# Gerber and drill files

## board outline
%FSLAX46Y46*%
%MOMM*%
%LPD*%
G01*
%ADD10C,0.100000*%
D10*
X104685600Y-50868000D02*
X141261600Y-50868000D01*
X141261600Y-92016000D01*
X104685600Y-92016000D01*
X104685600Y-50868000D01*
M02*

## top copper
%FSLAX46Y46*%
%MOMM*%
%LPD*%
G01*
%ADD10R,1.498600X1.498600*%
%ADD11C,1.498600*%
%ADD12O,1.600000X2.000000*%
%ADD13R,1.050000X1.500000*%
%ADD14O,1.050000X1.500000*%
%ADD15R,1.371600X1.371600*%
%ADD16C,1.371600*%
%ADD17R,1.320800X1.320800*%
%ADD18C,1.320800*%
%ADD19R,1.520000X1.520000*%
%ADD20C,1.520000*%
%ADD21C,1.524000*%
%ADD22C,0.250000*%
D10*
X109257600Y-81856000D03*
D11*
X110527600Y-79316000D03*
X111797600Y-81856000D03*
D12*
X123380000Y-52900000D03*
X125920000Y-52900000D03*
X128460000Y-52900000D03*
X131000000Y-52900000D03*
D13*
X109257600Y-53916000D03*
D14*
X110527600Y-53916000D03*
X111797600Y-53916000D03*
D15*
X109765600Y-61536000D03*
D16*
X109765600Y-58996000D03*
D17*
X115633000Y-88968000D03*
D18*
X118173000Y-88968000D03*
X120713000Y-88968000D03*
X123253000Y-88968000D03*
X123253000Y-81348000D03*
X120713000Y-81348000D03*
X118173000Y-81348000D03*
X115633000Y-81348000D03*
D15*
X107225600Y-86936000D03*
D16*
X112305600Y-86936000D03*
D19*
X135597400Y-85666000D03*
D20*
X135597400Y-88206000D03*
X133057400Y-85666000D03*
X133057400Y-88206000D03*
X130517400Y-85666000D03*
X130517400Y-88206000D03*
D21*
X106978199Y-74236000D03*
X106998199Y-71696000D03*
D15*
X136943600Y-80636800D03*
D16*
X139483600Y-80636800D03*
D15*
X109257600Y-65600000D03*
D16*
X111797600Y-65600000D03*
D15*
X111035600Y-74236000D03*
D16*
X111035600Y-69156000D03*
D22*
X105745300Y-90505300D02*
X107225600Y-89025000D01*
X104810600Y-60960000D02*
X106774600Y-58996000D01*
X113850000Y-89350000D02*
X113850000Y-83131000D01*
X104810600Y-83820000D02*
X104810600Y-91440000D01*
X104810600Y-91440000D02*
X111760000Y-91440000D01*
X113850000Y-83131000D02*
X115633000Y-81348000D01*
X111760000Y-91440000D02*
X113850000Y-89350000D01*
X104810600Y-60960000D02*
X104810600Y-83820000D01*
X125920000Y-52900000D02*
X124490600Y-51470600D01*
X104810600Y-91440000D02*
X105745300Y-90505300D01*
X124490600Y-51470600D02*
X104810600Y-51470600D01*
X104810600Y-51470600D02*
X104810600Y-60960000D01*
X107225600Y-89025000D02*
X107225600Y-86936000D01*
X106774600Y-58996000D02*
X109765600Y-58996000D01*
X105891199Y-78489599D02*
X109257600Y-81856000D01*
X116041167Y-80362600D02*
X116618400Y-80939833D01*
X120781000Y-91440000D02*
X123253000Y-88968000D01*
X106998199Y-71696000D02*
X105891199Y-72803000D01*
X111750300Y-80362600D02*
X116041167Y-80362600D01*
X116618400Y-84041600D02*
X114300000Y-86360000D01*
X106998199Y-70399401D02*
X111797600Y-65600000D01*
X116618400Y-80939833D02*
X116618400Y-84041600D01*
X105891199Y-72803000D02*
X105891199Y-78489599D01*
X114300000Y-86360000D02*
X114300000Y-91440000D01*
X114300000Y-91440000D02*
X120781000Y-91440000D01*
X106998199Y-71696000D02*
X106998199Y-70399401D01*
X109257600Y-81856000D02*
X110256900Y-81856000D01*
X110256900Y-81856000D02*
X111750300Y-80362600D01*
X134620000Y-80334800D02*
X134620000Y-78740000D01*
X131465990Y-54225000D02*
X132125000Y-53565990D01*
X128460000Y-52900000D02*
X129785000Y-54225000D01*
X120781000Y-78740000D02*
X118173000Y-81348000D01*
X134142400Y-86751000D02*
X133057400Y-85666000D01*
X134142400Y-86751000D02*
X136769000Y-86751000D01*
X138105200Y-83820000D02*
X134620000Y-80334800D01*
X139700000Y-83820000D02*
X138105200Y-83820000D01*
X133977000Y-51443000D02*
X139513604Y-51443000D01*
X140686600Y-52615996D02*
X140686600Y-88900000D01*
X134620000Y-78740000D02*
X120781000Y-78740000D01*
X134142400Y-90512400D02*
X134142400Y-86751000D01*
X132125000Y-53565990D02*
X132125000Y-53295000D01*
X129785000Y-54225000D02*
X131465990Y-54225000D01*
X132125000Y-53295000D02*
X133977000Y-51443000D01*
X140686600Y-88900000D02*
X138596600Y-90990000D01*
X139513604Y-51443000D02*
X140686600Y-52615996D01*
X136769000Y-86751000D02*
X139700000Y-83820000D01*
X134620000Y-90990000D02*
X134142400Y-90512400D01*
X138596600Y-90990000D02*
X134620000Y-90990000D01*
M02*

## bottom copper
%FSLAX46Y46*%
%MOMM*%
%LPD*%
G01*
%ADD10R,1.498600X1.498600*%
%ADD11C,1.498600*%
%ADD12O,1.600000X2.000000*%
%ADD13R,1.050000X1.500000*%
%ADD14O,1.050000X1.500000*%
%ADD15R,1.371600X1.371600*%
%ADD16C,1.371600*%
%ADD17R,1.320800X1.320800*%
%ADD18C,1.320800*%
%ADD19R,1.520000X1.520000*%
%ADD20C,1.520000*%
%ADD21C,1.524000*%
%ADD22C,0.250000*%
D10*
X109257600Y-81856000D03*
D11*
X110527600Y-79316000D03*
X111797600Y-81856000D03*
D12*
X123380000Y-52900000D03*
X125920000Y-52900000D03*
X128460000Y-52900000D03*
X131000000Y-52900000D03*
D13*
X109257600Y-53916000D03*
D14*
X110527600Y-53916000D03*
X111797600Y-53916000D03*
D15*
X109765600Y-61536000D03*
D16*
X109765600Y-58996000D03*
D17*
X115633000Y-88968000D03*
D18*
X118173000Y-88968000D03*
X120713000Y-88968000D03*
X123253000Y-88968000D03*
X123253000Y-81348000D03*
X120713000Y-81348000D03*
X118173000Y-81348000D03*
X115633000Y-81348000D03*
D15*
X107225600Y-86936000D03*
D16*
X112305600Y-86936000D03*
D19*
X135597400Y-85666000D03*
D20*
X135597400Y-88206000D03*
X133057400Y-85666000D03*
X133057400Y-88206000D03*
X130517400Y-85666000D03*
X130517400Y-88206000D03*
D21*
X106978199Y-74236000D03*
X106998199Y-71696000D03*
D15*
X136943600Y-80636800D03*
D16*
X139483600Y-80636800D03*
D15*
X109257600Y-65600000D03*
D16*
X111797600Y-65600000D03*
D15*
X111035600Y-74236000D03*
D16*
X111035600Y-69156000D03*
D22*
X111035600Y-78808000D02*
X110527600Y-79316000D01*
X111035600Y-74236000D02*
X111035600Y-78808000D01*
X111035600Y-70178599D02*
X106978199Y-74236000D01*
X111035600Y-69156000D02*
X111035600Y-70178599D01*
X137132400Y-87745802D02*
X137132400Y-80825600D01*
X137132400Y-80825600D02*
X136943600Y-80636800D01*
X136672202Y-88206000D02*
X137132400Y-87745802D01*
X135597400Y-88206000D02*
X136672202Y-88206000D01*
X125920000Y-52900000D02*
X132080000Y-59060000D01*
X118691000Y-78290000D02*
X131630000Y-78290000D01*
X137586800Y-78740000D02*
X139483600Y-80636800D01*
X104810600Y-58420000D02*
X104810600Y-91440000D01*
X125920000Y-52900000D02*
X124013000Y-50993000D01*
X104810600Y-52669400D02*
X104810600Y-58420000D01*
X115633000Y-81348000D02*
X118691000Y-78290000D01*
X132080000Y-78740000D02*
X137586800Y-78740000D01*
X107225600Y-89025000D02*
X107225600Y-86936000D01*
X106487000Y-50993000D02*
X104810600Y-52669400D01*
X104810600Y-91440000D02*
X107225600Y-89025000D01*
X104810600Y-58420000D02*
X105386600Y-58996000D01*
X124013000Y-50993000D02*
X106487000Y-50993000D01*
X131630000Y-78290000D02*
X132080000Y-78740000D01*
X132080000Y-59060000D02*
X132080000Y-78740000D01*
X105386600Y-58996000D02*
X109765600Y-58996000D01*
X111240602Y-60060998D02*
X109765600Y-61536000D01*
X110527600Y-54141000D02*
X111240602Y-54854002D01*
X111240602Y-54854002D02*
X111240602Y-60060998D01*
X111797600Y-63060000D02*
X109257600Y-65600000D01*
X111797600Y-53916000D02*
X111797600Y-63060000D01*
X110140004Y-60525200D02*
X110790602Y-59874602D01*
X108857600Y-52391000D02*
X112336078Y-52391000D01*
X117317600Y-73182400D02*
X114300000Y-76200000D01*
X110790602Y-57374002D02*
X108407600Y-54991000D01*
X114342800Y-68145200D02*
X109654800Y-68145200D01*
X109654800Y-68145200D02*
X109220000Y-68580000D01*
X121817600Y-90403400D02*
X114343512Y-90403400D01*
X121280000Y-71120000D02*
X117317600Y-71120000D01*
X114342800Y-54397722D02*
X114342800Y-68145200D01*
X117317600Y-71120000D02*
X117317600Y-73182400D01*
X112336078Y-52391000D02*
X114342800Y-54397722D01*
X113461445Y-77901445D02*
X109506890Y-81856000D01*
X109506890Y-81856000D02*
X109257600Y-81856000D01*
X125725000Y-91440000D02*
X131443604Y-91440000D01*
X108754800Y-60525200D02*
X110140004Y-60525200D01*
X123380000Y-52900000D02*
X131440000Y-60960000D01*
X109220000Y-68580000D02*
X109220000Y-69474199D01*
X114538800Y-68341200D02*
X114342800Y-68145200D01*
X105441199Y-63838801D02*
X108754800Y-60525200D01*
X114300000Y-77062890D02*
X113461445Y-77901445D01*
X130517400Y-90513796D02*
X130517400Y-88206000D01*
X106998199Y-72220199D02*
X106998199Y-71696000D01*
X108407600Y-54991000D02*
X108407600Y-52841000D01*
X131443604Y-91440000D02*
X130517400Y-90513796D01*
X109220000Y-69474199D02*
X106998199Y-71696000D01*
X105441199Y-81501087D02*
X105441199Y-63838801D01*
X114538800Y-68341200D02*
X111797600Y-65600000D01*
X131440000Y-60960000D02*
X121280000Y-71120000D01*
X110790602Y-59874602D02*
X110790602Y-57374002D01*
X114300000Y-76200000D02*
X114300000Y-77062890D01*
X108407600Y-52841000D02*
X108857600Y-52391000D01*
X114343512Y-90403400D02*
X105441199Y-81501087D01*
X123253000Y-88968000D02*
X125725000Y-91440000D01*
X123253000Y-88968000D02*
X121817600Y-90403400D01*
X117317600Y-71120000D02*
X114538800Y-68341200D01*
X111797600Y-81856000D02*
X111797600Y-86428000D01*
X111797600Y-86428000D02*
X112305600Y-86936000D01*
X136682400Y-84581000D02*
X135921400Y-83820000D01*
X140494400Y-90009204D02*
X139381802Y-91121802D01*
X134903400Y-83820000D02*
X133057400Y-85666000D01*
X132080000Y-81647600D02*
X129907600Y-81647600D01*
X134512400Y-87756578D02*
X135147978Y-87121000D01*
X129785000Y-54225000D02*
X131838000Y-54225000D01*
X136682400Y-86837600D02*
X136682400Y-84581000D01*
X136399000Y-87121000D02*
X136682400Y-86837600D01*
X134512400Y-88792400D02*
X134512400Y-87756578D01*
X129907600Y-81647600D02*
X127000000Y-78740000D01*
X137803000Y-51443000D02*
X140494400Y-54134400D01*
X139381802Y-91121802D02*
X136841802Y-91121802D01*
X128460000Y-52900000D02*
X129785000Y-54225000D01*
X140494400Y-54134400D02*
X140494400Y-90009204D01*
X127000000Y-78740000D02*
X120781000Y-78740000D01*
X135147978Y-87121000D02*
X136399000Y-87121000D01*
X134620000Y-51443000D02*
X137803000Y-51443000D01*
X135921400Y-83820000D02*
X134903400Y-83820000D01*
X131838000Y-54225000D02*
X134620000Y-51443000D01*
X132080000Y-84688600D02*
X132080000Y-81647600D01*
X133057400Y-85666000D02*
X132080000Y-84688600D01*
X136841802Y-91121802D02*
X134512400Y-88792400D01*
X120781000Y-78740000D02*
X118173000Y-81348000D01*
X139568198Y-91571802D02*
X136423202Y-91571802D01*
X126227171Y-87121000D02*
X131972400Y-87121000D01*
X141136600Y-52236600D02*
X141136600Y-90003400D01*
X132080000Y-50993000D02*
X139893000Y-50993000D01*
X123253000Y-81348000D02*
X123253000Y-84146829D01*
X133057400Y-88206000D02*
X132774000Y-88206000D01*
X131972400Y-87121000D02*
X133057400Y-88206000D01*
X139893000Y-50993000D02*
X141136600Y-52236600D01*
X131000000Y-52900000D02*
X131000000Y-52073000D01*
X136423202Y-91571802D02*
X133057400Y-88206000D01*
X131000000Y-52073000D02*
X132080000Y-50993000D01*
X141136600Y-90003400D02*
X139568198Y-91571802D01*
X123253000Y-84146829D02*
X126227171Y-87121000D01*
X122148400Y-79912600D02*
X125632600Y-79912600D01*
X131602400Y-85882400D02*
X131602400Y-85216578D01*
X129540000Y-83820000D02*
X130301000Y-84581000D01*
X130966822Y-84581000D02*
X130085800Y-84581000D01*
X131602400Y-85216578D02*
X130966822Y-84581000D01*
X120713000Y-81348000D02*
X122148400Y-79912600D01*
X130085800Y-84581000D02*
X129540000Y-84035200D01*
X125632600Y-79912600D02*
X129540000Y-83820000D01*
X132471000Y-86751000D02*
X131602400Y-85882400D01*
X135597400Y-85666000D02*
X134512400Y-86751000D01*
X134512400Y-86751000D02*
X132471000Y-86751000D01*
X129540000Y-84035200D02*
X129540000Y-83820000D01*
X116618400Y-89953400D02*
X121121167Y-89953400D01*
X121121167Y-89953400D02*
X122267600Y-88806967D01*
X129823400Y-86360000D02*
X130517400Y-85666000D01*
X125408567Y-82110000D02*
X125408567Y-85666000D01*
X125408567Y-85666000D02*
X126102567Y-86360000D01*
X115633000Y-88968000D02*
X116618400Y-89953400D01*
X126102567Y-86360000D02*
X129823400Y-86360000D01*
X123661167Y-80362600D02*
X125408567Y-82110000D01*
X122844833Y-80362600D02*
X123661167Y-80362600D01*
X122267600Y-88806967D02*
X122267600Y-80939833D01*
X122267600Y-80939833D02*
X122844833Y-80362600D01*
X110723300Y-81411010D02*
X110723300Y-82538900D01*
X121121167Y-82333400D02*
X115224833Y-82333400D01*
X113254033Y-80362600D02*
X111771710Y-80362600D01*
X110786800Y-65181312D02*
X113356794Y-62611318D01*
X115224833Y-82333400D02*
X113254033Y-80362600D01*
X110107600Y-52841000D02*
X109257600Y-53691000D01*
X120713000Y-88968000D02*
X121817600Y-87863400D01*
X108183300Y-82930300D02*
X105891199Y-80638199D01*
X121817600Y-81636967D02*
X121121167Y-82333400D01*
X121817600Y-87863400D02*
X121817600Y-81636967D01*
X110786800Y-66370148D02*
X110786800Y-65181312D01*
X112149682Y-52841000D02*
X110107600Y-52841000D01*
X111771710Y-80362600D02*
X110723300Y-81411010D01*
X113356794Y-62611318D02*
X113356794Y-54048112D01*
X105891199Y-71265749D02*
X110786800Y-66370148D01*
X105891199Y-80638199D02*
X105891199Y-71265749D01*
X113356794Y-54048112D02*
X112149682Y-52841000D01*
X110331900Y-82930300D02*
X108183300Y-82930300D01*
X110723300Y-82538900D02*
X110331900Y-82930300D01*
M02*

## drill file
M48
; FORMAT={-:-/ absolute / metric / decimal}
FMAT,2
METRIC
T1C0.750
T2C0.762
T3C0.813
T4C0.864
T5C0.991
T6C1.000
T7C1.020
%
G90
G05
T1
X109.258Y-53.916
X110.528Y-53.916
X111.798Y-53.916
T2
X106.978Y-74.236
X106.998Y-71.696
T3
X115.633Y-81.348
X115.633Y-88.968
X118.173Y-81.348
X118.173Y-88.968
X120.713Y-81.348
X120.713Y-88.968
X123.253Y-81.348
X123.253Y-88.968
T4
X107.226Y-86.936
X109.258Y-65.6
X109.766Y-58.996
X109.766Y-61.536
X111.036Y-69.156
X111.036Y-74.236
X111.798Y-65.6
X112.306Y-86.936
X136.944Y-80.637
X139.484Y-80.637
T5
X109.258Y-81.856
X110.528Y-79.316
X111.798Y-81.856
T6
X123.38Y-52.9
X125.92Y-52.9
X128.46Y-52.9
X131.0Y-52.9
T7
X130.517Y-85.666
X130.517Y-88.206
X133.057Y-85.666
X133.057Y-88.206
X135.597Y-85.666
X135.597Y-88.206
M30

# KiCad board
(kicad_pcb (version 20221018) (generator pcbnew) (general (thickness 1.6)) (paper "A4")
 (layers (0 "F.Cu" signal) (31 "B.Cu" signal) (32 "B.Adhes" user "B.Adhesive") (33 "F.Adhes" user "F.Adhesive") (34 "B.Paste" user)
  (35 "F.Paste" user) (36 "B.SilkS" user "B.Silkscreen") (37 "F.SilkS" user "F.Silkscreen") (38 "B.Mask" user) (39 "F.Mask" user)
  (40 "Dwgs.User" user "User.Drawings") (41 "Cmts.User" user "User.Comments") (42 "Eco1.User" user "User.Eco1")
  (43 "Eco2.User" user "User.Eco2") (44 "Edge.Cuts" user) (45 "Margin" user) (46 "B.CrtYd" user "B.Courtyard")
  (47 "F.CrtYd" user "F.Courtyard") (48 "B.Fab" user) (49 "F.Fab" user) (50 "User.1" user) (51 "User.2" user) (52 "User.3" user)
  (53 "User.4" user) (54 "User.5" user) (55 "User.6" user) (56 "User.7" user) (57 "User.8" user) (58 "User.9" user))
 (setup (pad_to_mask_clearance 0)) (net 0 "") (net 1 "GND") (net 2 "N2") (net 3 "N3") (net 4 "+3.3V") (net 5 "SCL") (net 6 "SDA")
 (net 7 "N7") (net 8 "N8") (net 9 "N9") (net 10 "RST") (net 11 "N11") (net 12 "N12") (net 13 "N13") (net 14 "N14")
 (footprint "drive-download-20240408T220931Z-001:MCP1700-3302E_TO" (layer "F.Cu") (at 111.7976 79.316)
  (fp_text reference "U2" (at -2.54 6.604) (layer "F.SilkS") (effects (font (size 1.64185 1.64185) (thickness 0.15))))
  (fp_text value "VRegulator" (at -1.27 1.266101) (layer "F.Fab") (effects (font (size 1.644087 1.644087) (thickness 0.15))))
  (pad "1" thru_hole rect (at -2.54 2.54) (size 1.4986 1.4986) (drill 0.9906) (layers "*.Cu" "*.Mask") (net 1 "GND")
   (solder_mask_margin 0.102))
  (pad "2" thru_hole circle (at -1.27 0) (size 1.4986 1.4986) (drill 0.9906) (layers "*.Cu" "*.Mask") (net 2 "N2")
   (solder_mask_margin 0.102))
  (pad "3" thru_hole circle (at 0 2.54) (size 1.4986 1.4986) (drill 0.9906) (layers "*.Cu" "*.Mask") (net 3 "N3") (solder_mask_margin 0.102)))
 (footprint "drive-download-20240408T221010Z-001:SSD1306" (layer "F.Cu") (at 127 63.5)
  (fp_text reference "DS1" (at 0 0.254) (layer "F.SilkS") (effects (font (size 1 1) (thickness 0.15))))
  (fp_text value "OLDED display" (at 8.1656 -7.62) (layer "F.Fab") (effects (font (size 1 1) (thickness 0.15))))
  (pad "1" thru_hole oval (at -3.62 -10.6 90) (size 2 1.6) (drill 1) (layers "*.Cu" "*.Mask") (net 1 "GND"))
  (pad "2" thru_hole oval (at -1.08 -10.6 90) (size 2 1.6) (drill 1) (layers "*.Cu" "*.Mask") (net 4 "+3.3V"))
  (pad "3" thru_hole oval (at 1.46 -10.6 90) (size 2 1.6) (drill 1) (layers "*.Cu" "*.Mask") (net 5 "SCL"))
  (pad "4" thru_hole oval (at 4 -10.6 90) (size 2 1.6) (drill 1) (layers "*.Cu" "*.Mask") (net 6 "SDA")))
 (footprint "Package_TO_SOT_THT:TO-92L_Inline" (layer "F.Cu") (at 109.2576 53.916)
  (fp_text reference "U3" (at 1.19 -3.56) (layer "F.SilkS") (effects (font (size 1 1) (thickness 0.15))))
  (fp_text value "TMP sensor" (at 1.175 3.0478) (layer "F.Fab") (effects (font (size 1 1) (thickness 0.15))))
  (pad "1" thru_hole rect (at 0 0) (size 1.05 1.5) (drill 0.75) (layers "*.Cu" "*.Mask") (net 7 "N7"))
  (pad "2" thru_hole oval (at 1.27 0) (size 1.05 1.5) (drill 0.75) (layers "*.Cu" "*.Mask") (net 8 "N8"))
  (pad "3" thru_hole oval (at 2.54 0) (size 1.05 1.5) (drill 0.75) (layers "*.Cu" "*.Mask") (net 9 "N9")))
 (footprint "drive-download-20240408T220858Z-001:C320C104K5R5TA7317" (layer "F.Cu") (at 109.7656 61.536 90)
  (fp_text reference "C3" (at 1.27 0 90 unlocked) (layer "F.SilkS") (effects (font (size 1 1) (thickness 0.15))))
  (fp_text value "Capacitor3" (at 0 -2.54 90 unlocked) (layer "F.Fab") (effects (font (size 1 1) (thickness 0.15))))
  (pad "1" thru_hole rect (at 0 0 90) (size 1.3716 1.3716) (drill 0.8636) (layers "*.Cu" "*.Mask") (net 8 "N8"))
  (pad "2" thru_hole circle (at 2.54 0 90) (size 1.3716 1.3716) (drill 0.8636) (layers "*.Cu" "*.Mask") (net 4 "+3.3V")))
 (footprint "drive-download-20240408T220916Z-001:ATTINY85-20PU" (layer "F.Cu") (at 119.443 85.158 90)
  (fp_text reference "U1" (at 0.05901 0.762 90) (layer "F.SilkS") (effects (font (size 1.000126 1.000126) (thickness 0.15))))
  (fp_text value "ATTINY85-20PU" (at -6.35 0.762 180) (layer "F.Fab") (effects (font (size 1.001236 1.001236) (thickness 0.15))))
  (pad "1" thru_hole rect (at -3.81 -3.81 90) (size 1.3208 1.3208) (drill 0.8128) (layers "*.Cu" "*.Mask") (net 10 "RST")
   (solder_mask_margin 0.102))
  (pad "2" thru_hole circle (at -3.81 -1.27 90) (size 1.3208 1.3208) (drill 0.8128) (layers "*.Cu" "*.Mask") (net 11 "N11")
   (solder_mask_margin 0.102))
  (pad "3" thru_hole circle (at -3.81 1.27 90) (size 1.3208 1.3208) (drill 0.8128) (layers "*.Cu" "*.Mask") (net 7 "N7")
   (solder_mask_margin 0.102))
  (pad "4" thru_hole circle (at -3.81 3.81 90) (size 1.3208 1.3208) (drill 0.8128) (layers "*.Cu" "*.Mask") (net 1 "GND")
   (solder_mask_margin 0.102))
  (pad "5" thru_hole circle (at 3.81 3.81 90) (size 1.3208 1.3208) (drill 0.8128) (layers "*.Cu" "*.Mask") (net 6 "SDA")
   (solder_mask_margin 0.102))
  (pad "6" thru_hole circle (at 3.81 1.27 90) (size 1.3208 1.3208) (drill 0.8128) (layers "*.Cu" "*.Mask") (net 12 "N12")
   (solder_mask_margin 0.102))
  (pad "7" thru_hole circle (at 3.81 -1.27 90) (size 1.3208 1.3208) (drill 0.8128) (layers "*.Cu" "*.Mask") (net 5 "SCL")
   (solder_mask_margin 0.102))
  (pad "8" thru_hole circle (at 3.81 -3.81 90) (size 1.3208 1.3208) (drill 0.8128) (layers "*.Cu" "*.Mask") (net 4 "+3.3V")
   (solder_mask_margin 0.102)))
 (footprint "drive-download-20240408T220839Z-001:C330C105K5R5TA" (layer "F.Cu") (at 107.2256 86.936)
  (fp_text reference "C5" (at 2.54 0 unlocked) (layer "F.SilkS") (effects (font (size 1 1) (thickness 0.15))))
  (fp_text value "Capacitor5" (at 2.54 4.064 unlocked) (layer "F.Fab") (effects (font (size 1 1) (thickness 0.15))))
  (pad "1" thru_hole rect (at 0 0) (size 1.3716 1.3716) (drill 0.8636) (layers "*.Cu" "*.Mask") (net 4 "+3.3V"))
  (pad "2" thru_hole circle (at 5.08 0) (size 1.3716 1.3716) (drill 0.8636) (layers "*.Cu" "*.Mask") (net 3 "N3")))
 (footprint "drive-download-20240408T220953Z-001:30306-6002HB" (layer "F.Cu") (at 135.5974 85.666 -90)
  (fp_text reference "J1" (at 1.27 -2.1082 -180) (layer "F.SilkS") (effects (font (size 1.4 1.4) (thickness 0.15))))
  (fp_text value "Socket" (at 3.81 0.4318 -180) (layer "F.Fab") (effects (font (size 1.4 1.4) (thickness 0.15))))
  (pad "1" thru_hole rect (at 0 0 270) (size 1.52 1.52) (drill 1.02) (layers "*.Cu" "*.Mask") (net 12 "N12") (solder_mask_margin 0.102))
  (pad "2" thru_hole circle (at 2.54 0 270) (size 1.52 1.52) (drill 1.02) (layers "*.Cu" "*.Mask") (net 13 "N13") (solder_mask_margin 0.102))
  (pad "3" thru_hole circle (at 0 2.54 270) (size 1.52 1.52) (drill 1.02) (layers "*.Cu" "*.Mask") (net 5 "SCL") (solder_mask_margin 0.102))
  (pad "4" thru_hole circle (at 2.54 2.54 270) (size 1.52 1.52) (drill 1.02) (layers "*.Cu" "*.Mask") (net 6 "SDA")
   (solder_mask_margin 0.102))
  (pad "5" thru_hole circle (at 0 5.08 270) (size 1.52 1.52) (drill 1.02) (layers "*.Cu" "*.Mask") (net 10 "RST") (solder_mask_margin 0.102))
  (pad "6" thru_hole circle (at 2.54 5.08 270) (size 1.52 1.52) (drill 1.02) (layers "*.Cu" "*.Mask") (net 1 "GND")
   (solder_mask_margin 0.102)))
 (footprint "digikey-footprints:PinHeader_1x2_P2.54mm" (layer "F.Cu") (at 106.978199 74.236 90)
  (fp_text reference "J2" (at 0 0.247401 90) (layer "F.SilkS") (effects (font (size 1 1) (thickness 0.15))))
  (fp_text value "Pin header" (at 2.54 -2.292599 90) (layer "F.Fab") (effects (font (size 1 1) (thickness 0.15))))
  (pad "1" thru_hole circle (at 0 0 90) (size 1.524 1.524) (drill 0.762) (layers "*.Cu" "*.Mask") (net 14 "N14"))
  (pad "2" thru_hole circle (at 2.54 0.02 90) (size 1.524 1.524) (drill 0.762) (layers "*.Cu" "*.Mask") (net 1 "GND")))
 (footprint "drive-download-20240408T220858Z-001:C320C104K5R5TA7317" (layer "F.Cu") (at 136.9436 80.6368)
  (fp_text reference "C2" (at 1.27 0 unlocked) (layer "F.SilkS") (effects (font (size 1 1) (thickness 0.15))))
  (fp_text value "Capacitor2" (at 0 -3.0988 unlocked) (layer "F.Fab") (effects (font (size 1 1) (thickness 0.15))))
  (pad "1" thru_hole rect (at 0 0) (size 1.3716 1.3716) (drill 0.8636) (layers "*.Cu" "*.Mask") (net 13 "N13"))
  (pad "2" thru_hole circle (at 2.54 0) (size 1.3716 1.3716) (drill 0.8636) (layers "*.Cu" "*.Mask") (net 4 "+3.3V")))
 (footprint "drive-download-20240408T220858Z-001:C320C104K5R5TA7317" (layer "F.Cu") (at 109.2576 65.6)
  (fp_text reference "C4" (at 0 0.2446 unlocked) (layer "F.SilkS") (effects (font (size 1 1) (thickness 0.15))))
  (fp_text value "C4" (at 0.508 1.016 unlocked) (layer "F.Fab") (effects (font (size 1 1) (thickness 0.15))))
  (pad "1" thru_hole rect (at 0 0) (size 1.3716 1.3716) (drill 0.8636) (layers "*.Cu" "*.Mask") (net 9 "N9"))
  (pad "2" thru_hole circle (at 2.54 0) (size 1.3716 1.3716) (drill 0.8636) (layers "*.Cu" "*.Mask") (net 1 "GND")))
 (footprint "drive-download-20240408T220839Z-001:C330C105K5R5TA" (layer "F.Cu") (at 111.0356 74.236 90)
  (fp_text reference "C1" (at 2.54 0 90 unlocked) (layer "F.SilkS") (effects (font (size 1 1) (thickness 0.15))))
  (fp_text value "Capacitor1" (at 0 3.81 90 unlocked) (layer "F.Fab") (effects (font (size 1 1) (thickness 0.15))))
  (pad "1" thru_hole rect (at 0 0 90) (size 1.3716 1.3716) (drill 0.8636) (layers "*.Cu" "*.Mask") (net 2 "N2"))
  (pad "2" thru_hole circle (at 5.08 0 90) (size 1.3716 1.3716) (drill 0.8636) (layers "*.Cu" "*.Mask") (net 14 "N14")))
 (gr_rect (start 104.6856 50.868) (end 141.2616 92.016) (stroke (width 0.1) (type default)) (fill none) (layer "Edge.Cuts"))
 (segment (start 111.0356 78.808) (end 110.5276 79.316) (width 0.25) (layer "B.Cu") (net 2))
 (segment (start 111.0356 74.236) (end 111.0356 78.808) (width 0.25) (layer "B.Cu") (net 2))
 (segment (start 111.0356 70.178599) (end 106.978199 74.236) (width 0.25) (layer "B.Cu") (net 14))
 (segment (start 111.0356 69.156) (end 111.0356 70.178599) (width 0.25) (layer "B.Cu") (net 14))
 (segment (start 137.1324 87.745802) (end 137.1324 80.8256) (width 0.25) (layer "B.Cu") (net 13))
 (segment (start 137.1324 80.8256) (end 136.9436 80.6368) (width 0.25) (layer "B.Cu") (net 13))
 (segment (start 136.672202 88.206) (end 137.1324 87.745802) (width 0.25) (layer "B.Cu") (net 13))
 (segment (start 135.5974 88.206) (end 136.672202 88.206) (width 0.25) (layer "B.Cu") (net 13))
 (segment (start 105.7453 90.5053) (end 107.2256 89.025) (width 0.25) (layer "F.Cu") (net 4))
 (segment (start 104.8106 60.96) (end 106.7746 58.996) (width 0.25) (layer "F.Cu") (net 4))
 (segment (start 113.85 89.35) (end 113.85 83.131) (width 0.25) (layer "F.Cu") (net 4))
 (segment (start 104.8106 83.82) (end 104.8106 91.44) (width 0.25) (layer "F.Cu") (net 4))
 (segment (start 104.8106 91.44) (end 111.76 91.44) (width 0.25) (layer "F.Cu") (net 4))
 (segment (start 113.85 83.131) (end 115.633 81.348) (width 0.25) (layer "F.Cu") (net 4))
 (segment (start 111.76 91.44) (end 113.85 89.35) (width 0.25) (layer "F.Cu") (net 4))
 (segment (start 104.8106 60.96) (end 104.8106 83.82) (width 0.25) (layer "F.Cu") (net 4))
 (segment (start 125.92 52.9) (end 124.4906 51.4706) (width 0.25) (layer "F.Cu") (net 4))
 (segment (start 104.8106 91.44) (end 105.7453 90.5053) (width 0.25) (layer "F.Cu") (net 4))
 (segment (start 124.4906 51.4706) (end 104.8106 51.4706) (width 0.25) (layer "F.Cu") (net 4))
 (segment (start 104.8106 51.4706) (end 104.8106 60.96) (width 0.25) (layer "F.Cu") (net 4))
 (segment (start 107.2256 89.025) (end 107.2256 86.936) (width 0.25) (layer "F.Cu") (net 4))
 (segment (start 106.7746 58.996) (end 109.7656 58.996) (width 0.25) (layer "F.Cu") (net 4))
 (segment (start 125.92 52.9) (end 132.08 59.06) (width 0.25) (layer "B.Cu") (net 4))
 (segment (start 118.691 78.29) (end 131.63 78.29) (width 0.25) (layer "B.Cu") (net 4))
 (segment (start 137.5868 78.74) (end 139.4836 80.6368) (width 0.25) (layer "B.Cu") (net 4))
 (segment (start 104.8106 58.42) (end 104.8106 91.44) (width 0.25) (layer "B.Cu") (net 4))
 (segment (start 125.92 52.9) (end 124.013 50.993) (width 0.25) (layer "B.Cu") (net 4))
 (segment (start 104.8106 52.6694) (end 104.8106 58.42) (width 0.25) (layer "B.Cu") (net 4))
 (segment (start 115.633 81.348) (end 118.691 78.29) (width 0.25) (layer "B.Cu") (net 4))
 (segment (start 132.08 78.74) (end 137.5868 78.74) (width 0.25) (layer "B.Cu") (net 4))
 (segment (start 107.2256 89.025) (end 107.2256 86.936) (width 0.25) (layer "B.Cu") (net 4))
 (segment (start 106.487 50.993) (end 104.8106 52.6694) (width 0.25) (layer "B.Cu") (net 4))
 (segment (start 104.8106 91.44) (end 107.2256 89.025) (width 0.25) (layer "B.Cu") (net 4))
 (segment (start 104.8106 58.42) (end 105.3866 58.996) (width 0.25) (layer "B.Cu") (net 4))
 (segment (start 124.013 50.993) (end 106.487 50.993) (width 0.25) (layer "B.Cu") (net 4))
 (segment (start 131.63 78.29) (end 132.08 78.74) (width 0.25) (layer "B.Cu") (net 4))
 (segment (start 132.08 59.06) (end 132.08 78.74) (width 0.25) (layer "B.Cu") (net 4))
 (segment (start 105.3866 58.996) (end 109.7656 58.996) (width 0.25) (layer "B.Cu") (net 4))
 (segment (start 111.240602 60.060998) (end 109.7656 61.536) (width 0.25) (layer "B.Cu") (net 8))
 (segment (start 110.5276 54.141) (end 111.240602 54.854002) (width 0.25) (layer "B.Cu") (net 8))
 (segment (start 111.240602 54.854002) (end 111.240602 60.060998) (width 0.25) (layer "B.Cu") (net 8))
 (segment (start 111.7976 63.06) (end 109.2576 65.6) (width 0.25) (layer "B.Cu") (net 9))
 (segment (start 111.7976 53.916) (end 111.7976 63.06) (width 0.25) (layer "B.Cu") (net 9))
 (segment (start 105.891199 78.489599) (end 109.2576 81.856) (width 0.25) (layer "F.Cu") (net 1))
 (segment (start 116.041167 80.3626) (end 116.6184 80.939833) (width 0.25) (layer "F.Cu") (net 1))
 (segment (start 120.781 91.44) (end 123.253 88.968) (width 0.25) (layer "F.Cu") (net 1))
 (segment (start 106.998199 71.696) (end 105.891199 72.803) (width 0.25) (layer "F.Cu") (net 1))
 (segment (start 111.7503 80.3626) (end 116.041167 80.3626) (width 0.25) (layer "F.Cu") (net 1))
 (segment (start 116.6184 84.0416) (end 114.3 86.36) (width 0.25) (layer "F.Cu") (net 1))
 (segment (start 106.998199 70.399401) (end 111.7976 65.6) (width 0.25) (layer "F.Cu") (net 1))
 (segment (start 116.6184 80.939833) (end 116.6184 84.0416) (width 0.25) (layer "F.Cu") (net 1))
 (segment (start 105.891199 72.803) (end 105.891199 78.489599) (width 0.25) (layer "F.Cu") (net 1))
 (segment (start 114.3 86.36) (end 114.3 91.44) (width 0.25) (layer "F.Cu") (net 1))
 (segment (start 114.3 91.44) (end 120.781 91.44) (width 0.25) (layer "F.Cu") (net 1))
 (segment (start 106.998199 71.696) (end 106.998199 70.399401) (width 0.25) (layer "F.Cu") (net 1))
 (segment (start 109.2576 81.856) (end 110.2569 81.856) (width 0.25) (layer "F.Cu") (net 1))
 (segment (start 110.2569 81.856) (end 111.7503 80.3626) (width 0.25) (layer "F.Cu") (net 1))
 (segment (start 110.140004 60.5252) (end 110.790602 59.874602) (width 0.25) (layer "B.Cu") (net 1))
 (segment (start 108.8576 52.391) (end 112.336078 52.391) (width 0.25) (layer "B.Cu") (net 1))
 (segment (start 117.3176 73.1824) (end 114.3 76.2) (width 0.25) (layer "B.Cu") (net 1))
 (segment (start 110.790602 57.374002) (end 108.4076 54.991) (width 0.25) (layer "B.Cu") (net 1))
 (segment (start 114.3428 68.1452) (end 109.6548 68.1452) (width 0.25) (layer "B.Cu") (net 1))
 (segment (start 109.6548 68.1452) (end 109.22 68.58) (width 0.25) (layer "B.Cu") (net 1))
 (segment (start 121.8176 90.4034) (end 114.343512 90.4034) (width 0.25) (layer "B.Cu") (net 1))
 (segment (start 121.28 71.12) (end 117.3176 71.12) (width 0.25) (layer "B.Cu") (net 1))
 (segment (start 114.3428 54.397722) (end 114.3428 68.1452) (width 0.25) (layer "B.Cu") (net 1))
 (segment (start 117.3176 71.12) (end 117.3176 73.1824) (width 0.25) (layer "B.Cu") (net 1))
 (segment (start 112.336078 52.391) (end 114.3428 54.397722) (width 0.25) (layer "B.Cu") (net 1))
 (segment (start 113.461445 77.901445) (end 109.50689 81.856) (width 0.25) (layer "B.Cu") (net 1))
 (segment (start 109.50689 81.856) (end 109.2576 81.856) (width 0.25) (layer "B.Cu") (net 1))
 (segment (start 125.725 91.44) (end 131.443604 91.44) (width 0.25) (layer "B.Cu") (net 1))
 (segment (start 108.7548 60.5252) (end 110.140004 60.5252) (width 0.25) (layer "B.Cu") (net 1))
 (segment (start 123.38 52.9) (end 131.44 60.96) (width 0.25) (layer "B.Cu") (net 1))
 (segment (start 109.22 68.58) (end 109.22 69.474199) (width 0.25) (layer "B.Cu") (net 1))
 (segment (start 114.5388 68.3412) (end 114.3428 68.1452) (width 0.25) (layer "B.Cu") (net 1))
 (segment (start 105.441199 63.838801) (end 108.7548 60.5252) (width 0.25) (layer "B.Cu") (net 1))
 (segment (start 114.3 77.06289) (end 113.461445 77.901445) (width 0.25) (layer "B.Cu") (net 1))
 (segment (start 130.5174 90.513796) (end 130.5174 88.206) (width 0.25) (layer "B.Cu") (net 1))
 (segment (start 106.998199 72.220199) (end 106.998199 71.696) (width 0.25) (layer "B.Cu") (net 1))
 (segment (start 108.4076 54.991) (end 108.4076 52.841) (width 0.25) (layer "B.Cu") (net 1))
 (segment (start 131.443604 91.44) (end 130.5174 90.513796) (width 0.25) (layer "B.Cu") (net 1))
 (segment (start 109.22 69.474199) (end 106.998199 71.696) (width 0.25) (layer "B.Cu") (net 1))
 (segment (start 105.441199 81.501087) (end 105.441199 63.838801) (width 0.25) (layer "B.Cu") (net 1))
 (segment (start 114.5388 68.3412) (end 111.7976 65.6) (width 0.25) (layer "B.Cu") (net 1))
 (segment (start 131.44 60.96) (end 121.28 71.12) (width 0.25) (layer "B.Cu") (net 1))
 (segment (start 110.790602 59.874602) (end 110.790602 57.374002) (width 0.25) (layer "B.Cu") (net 1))
 (segment (start 114.3 76.2) (end 114.3 77.06289) (width 0.25) (layer "B.Cu") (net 1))
 (segment (start 108.4076 52.841) (end 108.8576 52.391) (width 0.25) (layer "B.Cu") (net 1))
 (segment (start 114.343512 90.4034) (end 105.441199 81.501087) (width 0.25) (layer "B.Cu") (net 1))
 (segment (start 123.253 88.968) (end 125.725 91.44) (width 0.25) (layer "B.Cu") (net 1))
 (segment (start 123.253 88.968) (end 121.8176 90.4034) (width 0.25) (layer "B.Cu") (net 1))
 (segment (start 117.3176 71.12) (end 114.5388 68.3412) (width 0.25) (layer "B.Cu") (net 1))
 (segment (start 111.7976 81.856) (end 111.7976 86.428) (width 0.25) (layer "B.Cu") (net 3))
 (segment (start 111.7976 86.428) (end 112.3056 86.936) (width 0.25) (layer "B.Cu") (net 3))
 (segment (start 134.62 80.3348) (end 134.62 78.74) (width 0.25) (layer "F.Cu") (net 5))
 (segment (start 131.46599 54.225) (end 132.125 53.56599) (width 0.25) (layer "F.Cu") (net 5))
 (segment (start 128.46 52.9) (end 129.785 54.225) (width 0.25) (layer "F.Cu") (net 5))
 (segment (start 120.781 78.74) (end 118.173 81.348) (width 0.25) (layer "F.Cu") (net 5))
 (segment (start 134.1424 86.751) (end 133.0574 85.666) (width 0.25) (layer "F.Cu") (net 5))
 (segment (start 134.1424 86.751) (end 136.769 86.751) (width 0.25) (layer "F.Cu") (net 5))
 (segment (start 138.1052 83.82) (end 134.62 80.3348) (width 0.25) (layer "F.Cu") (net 5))
 (segment (start 139.7 83.82) (end 138.1052 83.82) (width 0.25) (layer "F.Cu") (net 5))
 (segment (start 133.977 51.443) (end 139.513604 51.443) (width 0.25) (layer "F.Cu") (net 5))
 (segment (start 140.6866 52.615996) (end 140.6866 88.9) (width 0.25) (layer "F.Cu") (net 5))
 (segment (start 134.62 78.74) (end 120.781 78.74) (width 0.25) (layer "F.Cu") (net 5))
 (segment (start 134.1424 90.5124) (end 134.1424 86.751) (width 0.25) (layer "F.Cu") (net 5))
 (segment (start 132.125 53.56599) (end 132.125 53.295) (width 0.25) (layer "F.Cu") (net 5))
 (segment (start 129.785 54.225) (end 131.46599 54.225) (width 0.25) (layer "F.Cu") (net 5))
 (segment (start 132.125 53.295) (end 133.977 51.443) (width 0.25) (layer "F.Cu") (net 5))
 (segment (start 140.6866 88.9) (end 138.5966 90.99) (width 0.25) (layer "F.Cu") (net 5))
 (segment (start 139.513604 51.443) (end 140.6866 52.615996) (width 0.25) (layer "F.Cu") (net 5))
 (segment (start 136.769 86.751) (end 139.7 83.82) (width 0.25) (layer "F.Cu") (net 5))
 (segment (start 134.62 90.99) (end 134.1424 90.5124) (width 0.25) (layer "F.Cu") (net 5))
 (segment (start 138.5966 90.99) (end 134.62 90.99) (width 0.25) (layer "F.Cu") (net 5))
 (segment (start 136.6824 84.581) (end 135.9214 83.82) (width 0.25) (layer "B.Cu") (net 5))
 (segment (start 140.4944 90.009204) (end 139.381802 91.121802) (width 0.25) (layer "B.Cu") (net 5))
 (segment (start 134.9034 83.82) (end 133.0574 85.666) (width 0.25) (layer "B.Cu") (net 5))
 (segment (start 132.08 81.6476) (end 129.9076 81.6476) (width 0.25) (layer "B.Cu") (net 5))
 (segment (start 134.5124 87.756578) (end 135.147978 87.121) (width 0.25) (layer "B.Cu") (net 5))
 (segment (start 129.785 54.225) (end 131.838 54.225) (width 0.25) (layer "B.Cu") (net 5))
 (segment (start 136.6824 86.8376) (end 136.6824 84.581) (width 0.25) (layer "B.Cu") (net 5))
 (segment (start 136.399 87.121) (end 136.6824 86.8376) (width 0.25) (layer "B.Cu") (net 5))
 (segment (start 134.5124 88.7924) (end 134.5124 87.756578) (width 0.25) (layer "B.Cu") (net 5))
 (segment (start 129.9076 81.6476) (end 127 78.74) (width 0.25) (layer "B.Cu") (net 5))
 (segment (start 137.803 51.443) (end 140.4944 54.1344) (width 0.25) (layer "B.Cu") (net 5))
 (segment (start 139.381802 91.121802) (end 136.841802 91.121802) (width 0.25) (layer "B.Cu") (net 5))
 (segment (start 128.46 52.9) (end 129.785 54.225) (width 0.25) (layer "B.Cu") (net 5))
 (segment (start 140.4944 54.1344) (end 140.4944 90.009204) (width 0.25) (layer "B.Cu") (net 5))
 (segment (start 127 78.74) (end 120.781 78.74) (width 0.25) (layer "B.Cu") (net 5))
 (segment (start 135.147978 87.121) (end 136.399 87.121) (width 0.25) (layer "B.Cu") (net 5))
 (segment (start 134.62 51.443) (end 137.803 51.443) (width 0.25) (layer "B.Cu") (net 5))
 (segment (start 135.9214 83.82) (end 134.9034 83.82) (width 0.25) (layer "B.Cu") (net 5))
 (segment (start 131.838 54.225) (end 134.62 51.443) (width 0.25) (layer "B.Cu") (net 5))
 (segment (start 132.08 84.6886) (end 132.08 81.6476) (width 0.25) (layer "B.Cu") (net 5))
 (segment (start 133.0574 85.666) (end 132.08 84.6886) (width 0.25) (layer "B.Cu") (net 5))
 (segment (start 136.841802 91.121802) (end 134.5124 88.7924) (width 0.25) (layer "B.Cu") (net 5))
 (segment (start 120.781 78.74) (end 118.173 81.348) (width 0.25) (layer "B.Cu") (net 5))
 (segment (start 139.568198 91.571802) (end 136.423202 91.571802) (width 0.25) (layer "B.Cu") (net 6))
 (segment (start 126.227171 87.121) (end 131.9724 87.121) (width 0.25) (layer "B.Cu") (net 6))
 (segment (start 141.1366 52.2366) (end 141.1366 90.0034) (width 0.25) (layer "B.Cu") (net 6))
 (segment (start 132.08 50.993) (end 139.893 50.993) (width 0.25) (layer "B.Cu") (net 6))
 (segment (start 123.253 81.348) (end 123.253 84.146829) (width 0.25) (layer "B.Cu") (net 6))
 (segment (start 133.0574 88.206) (end 132.774 88.206) (width 0.25) (layer "B.Cu") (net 6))
 (segment (start 131.9724 87.121) (end 133.0574 88.206) (width 0.25) (layer "B.Cu") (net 6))
 (segment (start 139.893 50.993) (end 141.1366 52.2366) (width 0.25) (layer "B.Cu") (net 6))
 (segment (start 131 52.9) (end 131 52.073) (width 0.25) (layer "B.Cu") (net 6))
 (segment (start 136.423202 91.571802) (end 133.0574 88.206) (width 0.25) (layer "B.Cu") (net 6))
 (segment (start 131 52.073) (end 132.08 50.993) (width 0.25) (layer "B.Cu") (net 6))
 (segment (start 141.1366 90.0034) (end 139.568198 91.571802) (width 0.25) (layer "B.Cu") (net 6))
 (segment (start 123.253 84.146829) (end 126.227171 87.121) (width 0.25) (layer "B.Cu") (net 6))
 (segment (start 122.1484 79.9126) (end 125.6326 79.9126) (width 0.25) (layer "B.Cu") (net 12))
 (segment (start 131.6024 85.8824) (end 131.6024 85.216578) (width 0.25) (layer "B.Cu") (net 12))
 (segment (start 129.54 83.82) (end 130.301 84.581) (width 0.25) (layer "B.Cu") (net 12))
 (segment (start 130.966822 84.581) (end 130.0858 84.581) (width 0.25) (layer "B.Cu") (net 12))
 (segment (start 131.6024 85.216578) (end 130.966822 84.581) (width 0.25) (layer "B.Cu") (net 12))
 (segment (start 120.713 81.348) (end 122.1484 79.9126) (width 0.25) (layer "B.Cu") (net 12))
 (segment (start 130.0858 84.581) (end 129.54 84.0352) (width 0.25) (layer "B.Cu") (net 12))
 (segment (start 125.6326 79.9126) (end 129.54 83.82) (width 0.25) (layer "B.Cu") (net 12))
 (segment (start 132.471 86.751) (end 131.6024 85.8824) (width 0.25) (layer "B.Cu") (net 12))
 (segment (start 135.5974 85.666) (end 134.5124 86.751) (width 0.25) (layer "B.Cu") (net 12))
 (segment (start 134.5124 86.751) (end 132.471 86.751) (width 0.25) (layer "B.Cu") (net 12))
 (segment (start 129.54 84.0352) (end 129.54 83.82) (width 0.25) (layer "B.Cu") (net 12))
 (segment (start 116.6184 89.9534) (end 121.121167 89.9534) (width 0.25) (layer "B.Cu") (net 10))
 (segment (start 121.121167 89.9534) (end 122.2676 88.806967) (width 0.25) (layer "B.Cu") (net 10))
 (segment (start 129.8234 86.36) (end 130.5174 85.666) (width 0.25) (layer "B.Cu") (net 10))
 (segment (start 125.408567 82.11) (end 125.408567 85.666) (width 0.25) (layer "B.Cu") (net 10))
 (segment (start 125.408567 85.666) (end 126.102567 86.36) (width 0.25) (layer "B.Cu") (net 10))
 (segment (start 115.633 88.968) (end 116.6184 89.9534) (width 0.25) (layer "B.Cu") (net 10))
 (segment (start 126.102567 86.36) (end 129.8234 86.36) (width 0.25) (layer "B.Cu") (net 10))
 (segment (start 123.661167 80.3626) (end 125.408567 82.11) (width 0.25) (layer "B.Cu") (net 10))
 (segment (start 122.844833 80.3626) (end 123.661167 80.3626) (width 0.25) (layer "B.Cu") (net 10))
 (segment (start 122.2676 88.806967) (end 122.2676 80.939833) (width 0.25) (layer "B.Cu") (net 10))
 (segment (start 122.2676 80.939833) (end 122.844833 80.3626) (width 0.25) (layer "B.Cu") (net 10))
 (segment (start 110.7233 81.41101) (end 110.7233 82.5389) (width 0.25) (layer "B.Cu") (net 7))
 (segment (start 121.121167 82.3334) (end 115.224833 82.3334) (width 0.25) (layer "B.Cu") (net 7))
 (segment (start 113.254033 80.3626) (end 111.77171 80.3626) (width 0.25) (layer "B.Cu") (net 7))
 (segment (start 110.7868 65.181312) (end 113.356794 62.611318) (width 0.25) (layer "B.Cu") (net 7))
 (segment (start 115.224833 82.3334) (end 113.254033 80.3626) (width 0.25) (layer "B.Cu") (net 7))
 (segment (start 110.1076 52.841) (end 109.2576 53.691) (width 0.25) (layer "B.Cu") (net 7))
 (segment (start 120.713 88.968) (end 121.8176 87.8634) (width 0.25) (layer "B.Cu") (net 7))
 (segment (start 108.1833 82.9303) (end 105.891199 80.638199) (width 0.25) (layer "B.Cu") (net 7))
 (segment (start 121.8176 81.636967) (end 121.121167 82.3334) (width 0.25) (layer "B.Cu") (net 7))
 (segment (start 121.8176 87.8634) (end 121.8176 81.636967) (width 0.25) (layer "B.Cu") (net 7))
 (segment (start 110.7868 66.370148) (end 110.7868 65.181312) (width 0.25) (layer "B.Cu") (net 7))
 (segment (start 112.149682 52.841) (end 110.1076 52.841) (width 0.25) (layer "B.Cu") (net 7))
 (segment (start 111.77171 80.3626) (end 110.7233 81.41101) (width 0.25) (layer "B.Cu") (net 7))
 (segment (start 113.356794 62.611318) (end 113.356794 54.048112) (width 0.25) (layer "B.Cu") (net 7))
 (segment (start 105.891199 71.265749) (end 110.7868 66.370148) (width 0.25) (layer "B.Cu") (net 7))
 (segment (start 105.891199 80.638199) (end 105.891199 71.265749) (width 0.25) (layer "B.Cu") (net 7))
 (segment (start 113.356794 54.048112) (end 112.149682 52.841) (width 0.25) (layer "B.Cu") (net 7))
 (segment (start 110.3319 82.9303) (end 108.1833 82.9303) (width 0.25) (layer "B.Cu") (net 7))
 (segment (start 110.7233 82.5389) (end 110.3319 82.9303) (width 0.25) (layer "B.Cu") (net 7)))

